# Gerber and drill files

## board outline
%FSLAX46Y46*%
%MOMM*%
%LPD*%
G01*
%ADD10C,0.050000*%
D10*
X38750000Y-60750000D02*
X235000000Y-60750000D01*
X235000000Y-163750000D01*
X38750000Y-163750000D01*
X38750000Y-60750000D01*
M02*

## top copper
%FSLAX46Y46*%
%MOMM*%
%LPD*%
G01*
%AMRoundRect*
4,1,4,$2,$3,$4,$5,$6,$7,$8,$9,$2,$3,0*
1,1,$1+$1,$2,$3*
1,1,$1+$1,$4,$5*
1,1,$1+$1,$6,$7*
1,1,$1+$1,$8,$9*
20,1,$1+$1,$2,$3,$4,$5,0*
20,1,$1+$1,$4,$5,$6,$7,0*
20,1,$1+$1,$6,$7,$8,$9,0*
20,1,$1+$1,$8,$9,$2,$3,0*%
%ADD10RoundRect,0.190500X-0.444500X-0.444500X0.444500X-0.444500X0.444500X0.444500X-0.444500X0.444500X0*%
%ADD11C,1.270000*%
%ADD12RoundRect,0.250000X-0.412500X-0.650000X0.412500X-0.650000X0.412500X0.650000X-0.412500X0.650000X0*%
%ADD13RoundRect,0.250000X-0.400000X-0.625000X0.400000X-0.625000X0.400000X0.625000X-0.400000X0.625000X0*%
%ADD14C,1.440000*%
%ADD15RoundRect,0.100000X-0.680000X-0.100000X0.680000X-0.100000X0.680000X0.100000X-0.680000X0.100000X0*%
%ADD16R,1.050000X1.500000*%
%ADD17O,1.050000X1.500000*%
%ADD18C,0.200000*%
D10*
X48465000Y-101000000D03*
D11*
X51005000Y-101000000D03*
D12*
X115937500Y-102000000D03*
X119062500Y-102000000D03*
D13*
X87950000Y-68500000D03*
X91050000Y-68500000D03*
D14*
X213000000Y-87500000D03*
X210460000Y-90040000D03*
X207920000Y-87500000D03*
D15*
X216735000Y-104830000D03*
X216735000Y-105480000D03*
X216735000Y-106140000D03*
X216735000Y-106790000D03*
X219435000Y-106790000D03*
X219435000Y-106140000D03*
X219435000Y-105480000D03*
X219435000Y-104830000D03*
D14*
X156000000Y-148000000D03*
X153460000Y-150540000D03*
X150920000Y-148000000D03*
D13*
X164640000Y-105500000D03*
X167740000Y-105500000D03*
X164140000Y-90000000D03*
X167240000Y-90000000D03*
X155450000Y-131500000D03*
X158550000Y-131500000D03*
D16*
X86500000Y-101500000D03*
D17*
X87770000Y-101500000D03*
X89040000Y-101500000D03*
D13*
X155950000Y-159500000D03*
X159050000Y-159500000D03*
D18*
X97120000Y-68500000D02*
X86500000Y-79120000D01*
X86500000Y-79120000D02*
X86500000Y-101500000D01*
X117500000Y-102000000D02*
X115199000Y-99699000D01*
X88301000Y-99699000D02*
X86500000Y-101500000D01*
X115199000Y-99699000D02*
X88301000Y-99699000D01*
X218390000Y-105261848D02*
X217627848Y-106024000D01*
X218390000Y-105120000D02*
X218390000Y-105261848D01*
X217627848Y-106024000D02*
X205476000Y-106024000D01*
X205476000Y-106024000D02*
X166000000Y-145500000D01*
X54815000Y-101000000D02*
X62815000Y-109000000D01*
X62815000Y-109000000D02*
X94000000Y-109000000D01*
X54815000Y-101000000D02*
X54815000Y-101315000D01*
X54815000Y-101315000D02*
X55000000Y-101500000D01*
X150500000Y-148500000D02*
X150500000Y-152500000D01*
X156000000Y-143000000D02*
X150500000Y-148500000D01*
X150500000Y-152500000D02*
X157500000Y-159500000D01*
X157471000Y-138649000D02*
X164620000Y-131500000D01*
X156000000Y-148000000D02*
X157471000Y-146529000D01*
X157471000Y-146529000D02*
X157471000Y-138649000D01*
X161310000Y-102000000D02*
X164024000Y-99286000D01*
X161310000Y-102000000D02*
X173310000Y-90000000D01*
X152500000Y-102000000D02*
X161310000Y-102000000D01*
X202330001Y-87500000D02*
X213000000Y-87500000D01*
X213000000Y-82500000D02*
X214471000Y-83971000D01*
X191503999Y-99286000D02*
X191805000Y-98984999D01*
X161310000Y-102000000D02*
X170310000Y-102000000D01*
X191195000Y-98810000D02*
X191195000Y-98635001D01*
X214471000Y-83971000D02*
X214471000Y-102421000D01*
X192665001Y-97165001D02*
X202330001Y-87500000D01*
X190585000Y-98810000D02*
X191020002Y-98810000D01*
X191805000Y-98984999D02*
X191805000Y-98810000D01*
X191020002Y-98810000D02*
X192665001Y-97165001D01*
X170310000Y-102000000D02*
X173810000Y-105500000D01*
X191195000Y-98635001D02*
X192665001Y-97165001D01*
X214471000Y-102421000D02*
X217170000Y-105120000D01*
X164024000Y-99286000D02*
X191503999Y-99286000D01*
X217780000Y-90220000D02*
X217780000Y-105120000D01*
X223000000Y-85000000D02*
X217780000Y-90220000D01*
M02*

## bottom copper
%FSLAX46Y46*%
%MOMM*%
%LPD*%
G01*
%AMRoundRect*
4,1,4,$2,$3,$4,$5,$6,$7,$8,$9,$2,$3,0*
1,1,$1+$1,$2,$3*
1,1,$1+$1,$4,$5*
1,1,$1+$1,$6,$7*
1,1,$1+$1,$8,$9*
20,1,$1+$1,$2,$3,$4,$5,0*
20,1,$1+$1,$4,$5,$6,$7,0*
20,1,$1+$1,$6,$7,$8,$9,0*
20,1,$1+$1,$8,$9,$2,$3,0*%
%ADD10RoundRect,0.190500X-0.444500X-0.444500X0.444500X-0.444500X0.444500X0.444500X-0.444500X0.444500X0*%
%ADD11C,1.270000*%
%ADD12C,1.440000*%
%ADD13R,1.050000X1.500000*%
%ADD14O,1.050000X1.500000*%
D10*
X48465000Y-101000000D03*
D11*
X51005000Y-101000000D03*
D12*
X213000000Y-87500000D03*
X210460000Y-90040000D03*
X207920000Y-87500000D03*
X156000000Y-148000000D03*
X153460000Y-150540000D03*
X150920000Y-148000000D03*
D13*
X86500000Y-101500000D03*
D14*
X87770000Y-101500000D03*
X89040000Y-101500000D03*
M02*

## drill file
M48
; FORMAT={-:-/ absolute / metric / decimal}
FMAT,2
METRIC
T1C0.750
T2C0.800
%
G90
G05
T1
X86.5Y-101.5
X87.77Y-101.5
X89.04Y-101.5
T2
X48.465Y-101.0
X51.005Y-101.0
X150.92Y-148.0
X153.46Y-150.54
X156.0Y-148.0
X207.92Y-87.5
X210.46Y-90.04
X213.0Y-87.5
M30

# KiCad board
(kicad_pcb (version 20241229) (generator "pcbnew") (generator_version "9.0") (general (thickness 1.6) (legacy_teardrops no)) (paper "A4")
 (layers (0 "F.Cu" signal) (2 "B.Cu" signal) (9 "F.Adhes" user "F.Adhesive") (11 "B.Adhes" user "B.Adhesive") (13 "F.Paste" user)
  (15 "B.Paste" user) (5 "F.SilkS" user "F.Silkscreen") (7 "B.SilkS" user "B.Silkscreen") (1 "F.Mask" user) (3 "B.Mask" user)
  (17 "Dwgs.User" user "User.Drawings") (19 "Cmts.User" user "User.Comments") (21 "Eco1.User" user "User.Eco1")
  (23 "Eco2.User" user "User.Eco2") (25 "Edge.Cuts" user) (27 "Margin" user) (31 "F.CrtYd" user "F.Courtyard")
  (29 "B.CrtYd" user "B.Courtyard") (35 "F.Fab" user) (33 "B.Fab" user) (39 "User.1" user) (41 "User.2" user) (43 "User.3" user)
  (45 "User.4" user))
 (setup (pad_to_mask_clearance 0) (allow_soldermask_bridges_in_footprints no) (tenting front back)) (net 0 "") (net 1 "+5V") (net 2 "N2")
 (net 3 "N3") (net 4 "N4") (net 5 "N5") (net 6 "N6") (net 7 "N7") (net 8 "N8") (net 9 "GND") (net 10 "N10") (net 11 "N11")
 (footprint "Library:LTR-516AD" (layer "F.Cu") (at 49.735 101)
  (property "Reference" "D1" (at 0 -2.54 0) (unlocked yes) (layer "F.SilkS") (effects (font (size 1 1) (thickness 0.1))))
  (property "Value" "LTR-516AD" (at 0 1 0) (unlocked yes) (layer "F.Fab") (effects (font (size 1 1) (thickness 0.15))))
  (pad "1" thru_hole roundrect (at -1.27 0) (size 1.27 1.27) (drill 0.8) (layers "*.Cu" "*.Mask") (remove_unused_layers no)
   (roundrect_rratio 0.15) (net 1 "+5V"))
  (pad "2" thru_hole circle (at 1.27 0) (size 1.27 1.27) (drill 0.8) (layers "*.Cu" "*.Mask") (remove_unused_layers no) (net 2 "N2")))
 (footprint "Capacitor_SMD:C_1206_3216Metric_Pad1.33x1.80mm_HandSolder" (layer "F.Cu") (at 117.5 102)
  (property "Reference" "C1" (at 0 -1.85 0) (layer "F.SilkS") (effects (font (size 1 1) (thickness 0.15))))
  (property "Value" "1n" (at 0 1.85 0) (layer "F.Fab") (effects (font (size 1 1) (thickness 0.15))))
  (pad "1" smd roundrect (at -1.5625 0) (size 1.325 1.8) (layers "F.Cu" "F.Mask" "F.Paste") (roundrect_rratio 0.188679) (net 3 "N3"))
  (pad "2" smd roundrect (at 1.5625 0) (size 1.325 1.8) (layers "F.Cu" "F.Mask" "F.Paste") (roundrect_rratio 0.188679) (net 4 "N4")))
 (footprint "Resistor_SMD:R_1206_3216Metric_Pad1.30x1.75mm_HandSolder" (layer "F.Cu") (at 89.5 68.5)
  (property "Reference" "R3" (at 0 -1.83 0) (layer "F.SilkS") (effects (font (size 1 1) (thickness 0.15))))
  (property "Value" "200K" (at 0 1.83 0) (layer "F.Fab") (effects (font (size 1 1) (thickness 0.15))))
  (pad "1" smd roundrect (at -1.55 0) (size 1.3 1.75) (layers "F.Cu" "F.Mask" "F.Paste") (roundrect_rratio 0.192308) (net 1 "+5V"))
  (pad "2" smd roundrect (at 1.55 0) (size 1.3 1.75) (layers "F.Cu" "F.Mask" "F.Paste") (roundrect_rratio 0.192308) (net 3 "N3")))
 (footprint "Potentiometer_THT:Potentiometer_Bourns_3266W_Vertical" (layer "F.Cu") (at 213 87.5)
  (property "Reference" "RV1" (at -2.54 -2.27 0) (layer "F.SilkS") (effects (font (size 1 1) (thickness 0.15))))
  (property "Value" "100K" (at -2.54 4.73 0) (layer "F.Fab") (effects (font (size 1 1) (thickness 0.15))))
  (pad "1" thru_hole circle (at 0 0) (size 1.44 1.44) (drill 0.8) (layers "*.Cu" "*.Mask") (remove_unused_layers no) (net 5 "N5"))
  (pad "2" thru_hole circle (at -2.54 2.54) (size 1.44 1.44) (drill 0.8) (layers "*.Cu" "*.Mask") (remove_unused_layers no) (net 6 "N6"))
  (pad "3" thru_hole circle (at -5.08 0) (size 1.44 1.44) (drill 0.8) (layers "*.Cu" "*.Mask") (remove_unused_layers no) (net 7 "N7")))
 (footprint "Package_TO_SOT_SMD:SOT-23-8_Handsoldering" (layer "F.Cu") (at 218.085 105.81)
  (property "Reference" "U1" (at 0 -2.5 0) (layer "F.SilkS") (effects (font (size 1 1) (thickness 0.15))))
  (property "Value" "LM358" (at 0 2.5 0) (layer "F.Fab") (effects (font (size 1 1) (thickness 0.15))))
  (pad "1" smd roundrect (at -1.35 -0.98) (size 1.56 0.4) (layers "F.Cu" "F.Mask" "F.Paste") (roundrect_rratio 0.25) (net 5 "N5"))
  (pad "2" smd roundrect (at -1.35 -0.33) (size 1.56 0.4) (layers "F.Cu" "F.Mask" "F.Paste") (roundrect_rratio 0.25) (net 5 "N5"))
  (pad "3" smd roundrect (at -1.35 0.33) (size 1.56 0.4) (layers "F.Cu" "F.Mask" "F.Paste") (roundrect_rratio 0.25) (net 4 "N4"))
  (pad "4" smd roundrect (at -1.35 0.98) (size 1.56 0.4) (layers "F.Cu" "F.Mask" "F.Paste") (roundrect_rratio 0.25) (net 1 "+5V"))
  (pad "5" smd roundrect (at 1.35 0.98) (size 1.56 0.4) (layers "F.Cu" "F.Mask" "F.Paste") (roundrect_rratio 0.25) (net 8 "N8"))
  (pad "6" smd roundrect (at 1.35 0.33) (size 1.56 0.4) (layers "F.Cu" "F.Mask" "F.Paste") (roundrect_rratio 0.25) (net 6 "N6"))
  (pad "7" smd roundrect (at 1.35 -0.33) (size 1.56 0.4) (layers "F.Cu" "F.Mask" "F.Paste") (roundrect_rratio 0.25) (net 7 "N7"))
  (pad "8" smd roundrect (at 1.35 -0.98) (size 1.56 0.4) (layers "F.Cu" "F.Mask" "F.Paste") (roundrect_rratio 0.25) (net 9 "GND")))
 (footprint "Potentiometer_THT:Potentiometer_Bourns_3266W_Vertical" (layer "F.Cu") (at 156 148)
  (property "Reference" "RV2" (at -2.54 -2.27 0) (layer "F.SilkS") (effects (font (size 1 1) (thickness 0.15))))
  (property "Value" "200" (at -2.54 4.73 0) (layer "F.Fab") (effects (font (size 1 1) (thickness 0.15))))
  (pad "1" thru_hole circle (at 0 0) (size 1.44 1.44) (drill 0.8) (layers "*.Cu" "*.Mask") (remove_unused_layers no) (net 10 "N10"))
  (pad "2" thru_hole circle (at -2.54 2.54) (size 1.44 1.44) (drill 0.8) (layers "*.Cu" "*.Mask") (remove_unused_layers no) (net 8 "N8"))
  (pad "3" thru_hole circle (at -5.08 0) (size 1.44 1.44) (drill 0.8) (layers "*.Cu" "*.Mask") (remove_unused_layers no) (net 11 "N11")))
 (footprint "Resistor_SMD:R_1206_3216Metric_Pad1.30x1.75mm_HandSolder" (layer "F.Cu") (at 166.19 105.5)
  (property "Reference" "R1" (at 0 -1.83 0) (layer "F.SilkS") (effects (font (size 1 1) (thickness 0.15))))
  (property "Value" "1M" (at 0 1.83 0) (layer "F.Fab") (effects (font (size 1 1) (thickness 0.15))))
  (pad "1" smd roundrect (at -1.55 0) (size 1.3 1.75) (layers "F.Cu" "F.Mask" "F.Paste") (roundrect_rratio 0.192308) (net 9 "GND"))
  (pad "2" smd roundrect (at 1.55 0) (size 1.3 1.75) (layers "F.Cu" "F.Mask" "F.Paste") (roundrect_rratio 0.192308) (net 4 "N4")))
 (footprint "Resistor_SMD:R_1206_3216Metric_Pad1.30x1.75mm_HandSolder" (layer "F.Cu") (at 165.69 90)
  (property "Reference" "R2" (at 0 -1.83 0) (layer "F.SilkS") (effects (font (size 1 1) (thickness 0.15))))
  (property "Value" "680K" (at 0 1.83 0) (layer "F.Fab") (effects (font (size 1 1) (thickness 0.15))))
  (pad "1" smd roundrect (at -1.55 0) (size 1.3 1.75) (layers "F.Cu" "F.Mask" "F.Paste") (roundrect_rratio 0.192308) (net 1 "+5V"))
  (pad "2" smd roundrect (at 1.55 0) (size 1.3 1.75) (layers "F.Cu" "F.Mask" "F.Paste") (roundrect_rratio 0.192308) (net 4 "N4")))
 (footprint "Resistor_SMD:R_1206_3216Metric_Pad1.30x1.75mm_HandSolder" (layer "F.Cu") (at 157 131.5)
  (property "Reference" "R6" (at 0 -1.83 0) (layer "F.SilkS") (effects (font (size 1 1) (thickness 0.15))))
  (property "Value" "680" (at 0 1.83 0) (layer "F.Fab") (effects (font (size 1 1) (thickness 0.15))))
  (pad "1" smd roundrect (at -1.55 0) (size 1.3 1.75) (layers "F.Cu" "F.Mask" "F.Paste") (roundrect_rratio 0.192308) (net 1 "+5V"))
  (pad "2" smd roundrect (at 1.55 0) (size 1.3 1.75) (layers "F.Cu" "F.Mask" "F.Paste") (roundrect_rratio 0.192308) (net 10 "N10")))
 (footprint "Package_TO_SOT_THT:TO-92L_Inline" (layer "F.Cu") (at 86.5 101.5)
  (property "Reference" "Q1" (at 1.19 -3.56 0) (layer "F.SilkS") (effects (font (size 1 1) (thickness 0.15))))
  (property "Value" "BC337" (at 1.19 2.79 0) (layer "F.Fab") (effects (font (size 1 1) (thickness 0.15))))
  (pad "1" thru_hole rect (at 0 0) (size 1.05 1.5) (drill 0.75) (layers "*.Cu" "*.Mask") (remove_unused_layers no) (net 3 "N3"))
  (pad "2" thru_hole oval (at 1.27 0) (size 1.05 1.5) (drill 0.75) (layers "*.Cu" "*.Mask") (remove_unused_layers no) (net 2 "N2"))
  (pad "3" thru_hole oval (at 2.54 0) (size 1.05 1.5) (drill 0.75) (layers "*.Cu" "*.Mask") (remove_unused_layers no) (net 9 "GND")))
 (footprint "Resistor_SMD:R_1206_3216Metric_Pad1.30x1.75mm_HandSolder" (layer "F.Cu") (at 157.5 159.5)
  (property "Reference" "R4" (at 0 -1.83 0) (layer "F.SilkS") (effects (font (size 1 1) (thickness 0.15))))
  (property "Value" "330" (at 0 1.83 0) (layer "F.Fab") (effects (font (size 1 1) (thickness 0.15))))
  (pad "1" smd roundrect (at -1.55 0) (size 1.3 1.75) (layers "F.Cu" "F.Mask" "F.Paste") (roundrect_rratio 0.192308) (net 11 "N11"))
  (pad "2" smd roundrect (at 1.55 0) (size 1.3 1.75) (layers "F.Cu" "F.Mask" "F.Paste") (roundrect_rratio 0.192308) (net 9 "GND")))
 (gr_rect (start 38.75 60.75) (end 235 163.75) (stroke (width 0.05) (type default)) (fill no) (layer "Edge.Cuts"))
 (segment (start 97.12 68.5) (end 86.5 79.12) (width 0.2) (layer "F.Cu") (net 3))
 (segment (start 86.5 79.12) (end 86.5 101.5) (width 0.2) (layer "F.Cu") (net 3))
 (segment (start 117.5 102) (end 115.199 99.699) (width 0.2) (layer "F.Cu") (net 3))
 (segment (start 88.301 99.699) (end 86.5 101.5) (width 0.2) (layer "F.Cu") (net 3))
 (segment (start 115.199 99.699) (end 88.301 99.699) (width 0.2) (layer "F.Cu") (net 3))
 (segment (start 218.39 105.261848) (end 217.627848 106.024) (width 0.2) (layer "F.Cu") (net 4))
 (segment (start 218.39 105.12) (end 218.39 105.261848) (width 0.2) (layer "F.Cu") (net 4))
 (segment (start 217.627848 106.024) (end 205.476 106.024) (width 0.2) (layer "F.Cu") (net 4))
 (segment (start 205.476 106.024) (end 166 145.5) (width 0.2) (layer "F.Cu") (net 4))
 (segment (start 54.815 101) (end 62.815 109) (width 0.2) (layer "F.Cu") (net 2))
 (segment (start 62.815 109) (end 94 109) (width 0.2) (layer "F.Cu") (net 2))
 (segment (start 54.815 101) (end 54.815 101.315) (width 0.2) (layer "F.Cu") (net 2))
 (segment (start 54.815 101.315) (end 55 101.5) (width 0.2) (layer "F.Cu") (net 2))
 (segment (start 150.5 148.5) (end 150.5 152.5) (width 0.2) (layer "F.Cu") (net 11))
 (segment (start 156 143) (end 150.5 148.5) (width 0.2) (layer "F.Cu") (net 11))
 (segment (start 150.5 152.5) (end 157.5 159.5) (width 0.2) (layer "F.Cu") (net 11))
 (segment (start 157.471 138.649) (end 164.62 131.5) (width 0.2) (layer "F.Cu") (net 10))
 (segment (start 156 148) (end 157.471 146.529) (width 0.2) (layer "F.Cu") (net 10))
 (segment (start 157.471 146.529) (end 157.471 138.649) (width 0.2) (layer "F.Cu") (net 10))
 (segment (start 161.31 102) (end 164.024 99.286) (width 0.2) (layer "F.Cu") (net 5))
 (segment (start 161.31 102) (end 173.31 90) (width 0.2) (layer "F.Cu") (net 5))
 (segment (start 152.5 102) (end 161.31 102) (width 0.2) (layer "F.Cu") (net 5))
 (segment (start 202.330001 87.5) (end 213 87.5) (width 0.2) (layer "F.Cu") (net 5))
 (segment (start 213 82.5) (end 214.471 83.971) (width 0.2) (layer "F.Cu") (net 5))
 (segment (start 191.503999 99.286) (end 191.805 98.984999) (width 0.2) (layer "F.Cu") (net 5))
 (segment (start 161.31 102) (end 170.31 102) (width 0.2) (layer "F.Cu") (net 5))
 (segment (start 191.195 98.81) (end 191.195 98.635001) (width 0.2) (layer "F.Cu") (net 5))
 (segment (start 214.471 83.971) (end 214.471 102.421) (width 0.2) (layer "F.Cu") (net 5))
 (segment (start 192.665001 97.165001) (end 202.330001 87.5) (width 0.2) (layer "F.Cu") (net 5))
 (segment (start 190.585 98.81) (end 191.020002 98.81) (width 0.2) (layer "F.Cu") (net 5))
 (segment (start 191.805 98.984999) (end 191.805 98.81) (width 0.2) (layer "F.Cu") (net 5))
 (segment (start 191.020002 98.81) (end 192.665001 97.165001) (width 0.2) (layer "F.Cu") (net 5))
 (segment (start 170.31 102) (end 173.81 105.5) (width 0.2) (layer "F.Cu") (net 5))
 (segment (start 191.195 98.635001) (end 192.665001 97.165001) (width 0.2) (layer "F.Cu") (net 5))
 (segment (start 214.471 102.421) (end 217.17 105.12) (width 0.2) (layer "F.Cu") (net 5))
 (segment (start 164.024 99.286) (end 191.503999 99.286) (width 0.2) (layer "F.Cu") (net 5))
 (segment (start 217.78 90.22) (end 217.78 105.12) (width 0.2) (layer "F.Cu") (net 6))
 (segment (start 223 85) (end 217.78 90.22) (width 0.2) (layer "F.Cu") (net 6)))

